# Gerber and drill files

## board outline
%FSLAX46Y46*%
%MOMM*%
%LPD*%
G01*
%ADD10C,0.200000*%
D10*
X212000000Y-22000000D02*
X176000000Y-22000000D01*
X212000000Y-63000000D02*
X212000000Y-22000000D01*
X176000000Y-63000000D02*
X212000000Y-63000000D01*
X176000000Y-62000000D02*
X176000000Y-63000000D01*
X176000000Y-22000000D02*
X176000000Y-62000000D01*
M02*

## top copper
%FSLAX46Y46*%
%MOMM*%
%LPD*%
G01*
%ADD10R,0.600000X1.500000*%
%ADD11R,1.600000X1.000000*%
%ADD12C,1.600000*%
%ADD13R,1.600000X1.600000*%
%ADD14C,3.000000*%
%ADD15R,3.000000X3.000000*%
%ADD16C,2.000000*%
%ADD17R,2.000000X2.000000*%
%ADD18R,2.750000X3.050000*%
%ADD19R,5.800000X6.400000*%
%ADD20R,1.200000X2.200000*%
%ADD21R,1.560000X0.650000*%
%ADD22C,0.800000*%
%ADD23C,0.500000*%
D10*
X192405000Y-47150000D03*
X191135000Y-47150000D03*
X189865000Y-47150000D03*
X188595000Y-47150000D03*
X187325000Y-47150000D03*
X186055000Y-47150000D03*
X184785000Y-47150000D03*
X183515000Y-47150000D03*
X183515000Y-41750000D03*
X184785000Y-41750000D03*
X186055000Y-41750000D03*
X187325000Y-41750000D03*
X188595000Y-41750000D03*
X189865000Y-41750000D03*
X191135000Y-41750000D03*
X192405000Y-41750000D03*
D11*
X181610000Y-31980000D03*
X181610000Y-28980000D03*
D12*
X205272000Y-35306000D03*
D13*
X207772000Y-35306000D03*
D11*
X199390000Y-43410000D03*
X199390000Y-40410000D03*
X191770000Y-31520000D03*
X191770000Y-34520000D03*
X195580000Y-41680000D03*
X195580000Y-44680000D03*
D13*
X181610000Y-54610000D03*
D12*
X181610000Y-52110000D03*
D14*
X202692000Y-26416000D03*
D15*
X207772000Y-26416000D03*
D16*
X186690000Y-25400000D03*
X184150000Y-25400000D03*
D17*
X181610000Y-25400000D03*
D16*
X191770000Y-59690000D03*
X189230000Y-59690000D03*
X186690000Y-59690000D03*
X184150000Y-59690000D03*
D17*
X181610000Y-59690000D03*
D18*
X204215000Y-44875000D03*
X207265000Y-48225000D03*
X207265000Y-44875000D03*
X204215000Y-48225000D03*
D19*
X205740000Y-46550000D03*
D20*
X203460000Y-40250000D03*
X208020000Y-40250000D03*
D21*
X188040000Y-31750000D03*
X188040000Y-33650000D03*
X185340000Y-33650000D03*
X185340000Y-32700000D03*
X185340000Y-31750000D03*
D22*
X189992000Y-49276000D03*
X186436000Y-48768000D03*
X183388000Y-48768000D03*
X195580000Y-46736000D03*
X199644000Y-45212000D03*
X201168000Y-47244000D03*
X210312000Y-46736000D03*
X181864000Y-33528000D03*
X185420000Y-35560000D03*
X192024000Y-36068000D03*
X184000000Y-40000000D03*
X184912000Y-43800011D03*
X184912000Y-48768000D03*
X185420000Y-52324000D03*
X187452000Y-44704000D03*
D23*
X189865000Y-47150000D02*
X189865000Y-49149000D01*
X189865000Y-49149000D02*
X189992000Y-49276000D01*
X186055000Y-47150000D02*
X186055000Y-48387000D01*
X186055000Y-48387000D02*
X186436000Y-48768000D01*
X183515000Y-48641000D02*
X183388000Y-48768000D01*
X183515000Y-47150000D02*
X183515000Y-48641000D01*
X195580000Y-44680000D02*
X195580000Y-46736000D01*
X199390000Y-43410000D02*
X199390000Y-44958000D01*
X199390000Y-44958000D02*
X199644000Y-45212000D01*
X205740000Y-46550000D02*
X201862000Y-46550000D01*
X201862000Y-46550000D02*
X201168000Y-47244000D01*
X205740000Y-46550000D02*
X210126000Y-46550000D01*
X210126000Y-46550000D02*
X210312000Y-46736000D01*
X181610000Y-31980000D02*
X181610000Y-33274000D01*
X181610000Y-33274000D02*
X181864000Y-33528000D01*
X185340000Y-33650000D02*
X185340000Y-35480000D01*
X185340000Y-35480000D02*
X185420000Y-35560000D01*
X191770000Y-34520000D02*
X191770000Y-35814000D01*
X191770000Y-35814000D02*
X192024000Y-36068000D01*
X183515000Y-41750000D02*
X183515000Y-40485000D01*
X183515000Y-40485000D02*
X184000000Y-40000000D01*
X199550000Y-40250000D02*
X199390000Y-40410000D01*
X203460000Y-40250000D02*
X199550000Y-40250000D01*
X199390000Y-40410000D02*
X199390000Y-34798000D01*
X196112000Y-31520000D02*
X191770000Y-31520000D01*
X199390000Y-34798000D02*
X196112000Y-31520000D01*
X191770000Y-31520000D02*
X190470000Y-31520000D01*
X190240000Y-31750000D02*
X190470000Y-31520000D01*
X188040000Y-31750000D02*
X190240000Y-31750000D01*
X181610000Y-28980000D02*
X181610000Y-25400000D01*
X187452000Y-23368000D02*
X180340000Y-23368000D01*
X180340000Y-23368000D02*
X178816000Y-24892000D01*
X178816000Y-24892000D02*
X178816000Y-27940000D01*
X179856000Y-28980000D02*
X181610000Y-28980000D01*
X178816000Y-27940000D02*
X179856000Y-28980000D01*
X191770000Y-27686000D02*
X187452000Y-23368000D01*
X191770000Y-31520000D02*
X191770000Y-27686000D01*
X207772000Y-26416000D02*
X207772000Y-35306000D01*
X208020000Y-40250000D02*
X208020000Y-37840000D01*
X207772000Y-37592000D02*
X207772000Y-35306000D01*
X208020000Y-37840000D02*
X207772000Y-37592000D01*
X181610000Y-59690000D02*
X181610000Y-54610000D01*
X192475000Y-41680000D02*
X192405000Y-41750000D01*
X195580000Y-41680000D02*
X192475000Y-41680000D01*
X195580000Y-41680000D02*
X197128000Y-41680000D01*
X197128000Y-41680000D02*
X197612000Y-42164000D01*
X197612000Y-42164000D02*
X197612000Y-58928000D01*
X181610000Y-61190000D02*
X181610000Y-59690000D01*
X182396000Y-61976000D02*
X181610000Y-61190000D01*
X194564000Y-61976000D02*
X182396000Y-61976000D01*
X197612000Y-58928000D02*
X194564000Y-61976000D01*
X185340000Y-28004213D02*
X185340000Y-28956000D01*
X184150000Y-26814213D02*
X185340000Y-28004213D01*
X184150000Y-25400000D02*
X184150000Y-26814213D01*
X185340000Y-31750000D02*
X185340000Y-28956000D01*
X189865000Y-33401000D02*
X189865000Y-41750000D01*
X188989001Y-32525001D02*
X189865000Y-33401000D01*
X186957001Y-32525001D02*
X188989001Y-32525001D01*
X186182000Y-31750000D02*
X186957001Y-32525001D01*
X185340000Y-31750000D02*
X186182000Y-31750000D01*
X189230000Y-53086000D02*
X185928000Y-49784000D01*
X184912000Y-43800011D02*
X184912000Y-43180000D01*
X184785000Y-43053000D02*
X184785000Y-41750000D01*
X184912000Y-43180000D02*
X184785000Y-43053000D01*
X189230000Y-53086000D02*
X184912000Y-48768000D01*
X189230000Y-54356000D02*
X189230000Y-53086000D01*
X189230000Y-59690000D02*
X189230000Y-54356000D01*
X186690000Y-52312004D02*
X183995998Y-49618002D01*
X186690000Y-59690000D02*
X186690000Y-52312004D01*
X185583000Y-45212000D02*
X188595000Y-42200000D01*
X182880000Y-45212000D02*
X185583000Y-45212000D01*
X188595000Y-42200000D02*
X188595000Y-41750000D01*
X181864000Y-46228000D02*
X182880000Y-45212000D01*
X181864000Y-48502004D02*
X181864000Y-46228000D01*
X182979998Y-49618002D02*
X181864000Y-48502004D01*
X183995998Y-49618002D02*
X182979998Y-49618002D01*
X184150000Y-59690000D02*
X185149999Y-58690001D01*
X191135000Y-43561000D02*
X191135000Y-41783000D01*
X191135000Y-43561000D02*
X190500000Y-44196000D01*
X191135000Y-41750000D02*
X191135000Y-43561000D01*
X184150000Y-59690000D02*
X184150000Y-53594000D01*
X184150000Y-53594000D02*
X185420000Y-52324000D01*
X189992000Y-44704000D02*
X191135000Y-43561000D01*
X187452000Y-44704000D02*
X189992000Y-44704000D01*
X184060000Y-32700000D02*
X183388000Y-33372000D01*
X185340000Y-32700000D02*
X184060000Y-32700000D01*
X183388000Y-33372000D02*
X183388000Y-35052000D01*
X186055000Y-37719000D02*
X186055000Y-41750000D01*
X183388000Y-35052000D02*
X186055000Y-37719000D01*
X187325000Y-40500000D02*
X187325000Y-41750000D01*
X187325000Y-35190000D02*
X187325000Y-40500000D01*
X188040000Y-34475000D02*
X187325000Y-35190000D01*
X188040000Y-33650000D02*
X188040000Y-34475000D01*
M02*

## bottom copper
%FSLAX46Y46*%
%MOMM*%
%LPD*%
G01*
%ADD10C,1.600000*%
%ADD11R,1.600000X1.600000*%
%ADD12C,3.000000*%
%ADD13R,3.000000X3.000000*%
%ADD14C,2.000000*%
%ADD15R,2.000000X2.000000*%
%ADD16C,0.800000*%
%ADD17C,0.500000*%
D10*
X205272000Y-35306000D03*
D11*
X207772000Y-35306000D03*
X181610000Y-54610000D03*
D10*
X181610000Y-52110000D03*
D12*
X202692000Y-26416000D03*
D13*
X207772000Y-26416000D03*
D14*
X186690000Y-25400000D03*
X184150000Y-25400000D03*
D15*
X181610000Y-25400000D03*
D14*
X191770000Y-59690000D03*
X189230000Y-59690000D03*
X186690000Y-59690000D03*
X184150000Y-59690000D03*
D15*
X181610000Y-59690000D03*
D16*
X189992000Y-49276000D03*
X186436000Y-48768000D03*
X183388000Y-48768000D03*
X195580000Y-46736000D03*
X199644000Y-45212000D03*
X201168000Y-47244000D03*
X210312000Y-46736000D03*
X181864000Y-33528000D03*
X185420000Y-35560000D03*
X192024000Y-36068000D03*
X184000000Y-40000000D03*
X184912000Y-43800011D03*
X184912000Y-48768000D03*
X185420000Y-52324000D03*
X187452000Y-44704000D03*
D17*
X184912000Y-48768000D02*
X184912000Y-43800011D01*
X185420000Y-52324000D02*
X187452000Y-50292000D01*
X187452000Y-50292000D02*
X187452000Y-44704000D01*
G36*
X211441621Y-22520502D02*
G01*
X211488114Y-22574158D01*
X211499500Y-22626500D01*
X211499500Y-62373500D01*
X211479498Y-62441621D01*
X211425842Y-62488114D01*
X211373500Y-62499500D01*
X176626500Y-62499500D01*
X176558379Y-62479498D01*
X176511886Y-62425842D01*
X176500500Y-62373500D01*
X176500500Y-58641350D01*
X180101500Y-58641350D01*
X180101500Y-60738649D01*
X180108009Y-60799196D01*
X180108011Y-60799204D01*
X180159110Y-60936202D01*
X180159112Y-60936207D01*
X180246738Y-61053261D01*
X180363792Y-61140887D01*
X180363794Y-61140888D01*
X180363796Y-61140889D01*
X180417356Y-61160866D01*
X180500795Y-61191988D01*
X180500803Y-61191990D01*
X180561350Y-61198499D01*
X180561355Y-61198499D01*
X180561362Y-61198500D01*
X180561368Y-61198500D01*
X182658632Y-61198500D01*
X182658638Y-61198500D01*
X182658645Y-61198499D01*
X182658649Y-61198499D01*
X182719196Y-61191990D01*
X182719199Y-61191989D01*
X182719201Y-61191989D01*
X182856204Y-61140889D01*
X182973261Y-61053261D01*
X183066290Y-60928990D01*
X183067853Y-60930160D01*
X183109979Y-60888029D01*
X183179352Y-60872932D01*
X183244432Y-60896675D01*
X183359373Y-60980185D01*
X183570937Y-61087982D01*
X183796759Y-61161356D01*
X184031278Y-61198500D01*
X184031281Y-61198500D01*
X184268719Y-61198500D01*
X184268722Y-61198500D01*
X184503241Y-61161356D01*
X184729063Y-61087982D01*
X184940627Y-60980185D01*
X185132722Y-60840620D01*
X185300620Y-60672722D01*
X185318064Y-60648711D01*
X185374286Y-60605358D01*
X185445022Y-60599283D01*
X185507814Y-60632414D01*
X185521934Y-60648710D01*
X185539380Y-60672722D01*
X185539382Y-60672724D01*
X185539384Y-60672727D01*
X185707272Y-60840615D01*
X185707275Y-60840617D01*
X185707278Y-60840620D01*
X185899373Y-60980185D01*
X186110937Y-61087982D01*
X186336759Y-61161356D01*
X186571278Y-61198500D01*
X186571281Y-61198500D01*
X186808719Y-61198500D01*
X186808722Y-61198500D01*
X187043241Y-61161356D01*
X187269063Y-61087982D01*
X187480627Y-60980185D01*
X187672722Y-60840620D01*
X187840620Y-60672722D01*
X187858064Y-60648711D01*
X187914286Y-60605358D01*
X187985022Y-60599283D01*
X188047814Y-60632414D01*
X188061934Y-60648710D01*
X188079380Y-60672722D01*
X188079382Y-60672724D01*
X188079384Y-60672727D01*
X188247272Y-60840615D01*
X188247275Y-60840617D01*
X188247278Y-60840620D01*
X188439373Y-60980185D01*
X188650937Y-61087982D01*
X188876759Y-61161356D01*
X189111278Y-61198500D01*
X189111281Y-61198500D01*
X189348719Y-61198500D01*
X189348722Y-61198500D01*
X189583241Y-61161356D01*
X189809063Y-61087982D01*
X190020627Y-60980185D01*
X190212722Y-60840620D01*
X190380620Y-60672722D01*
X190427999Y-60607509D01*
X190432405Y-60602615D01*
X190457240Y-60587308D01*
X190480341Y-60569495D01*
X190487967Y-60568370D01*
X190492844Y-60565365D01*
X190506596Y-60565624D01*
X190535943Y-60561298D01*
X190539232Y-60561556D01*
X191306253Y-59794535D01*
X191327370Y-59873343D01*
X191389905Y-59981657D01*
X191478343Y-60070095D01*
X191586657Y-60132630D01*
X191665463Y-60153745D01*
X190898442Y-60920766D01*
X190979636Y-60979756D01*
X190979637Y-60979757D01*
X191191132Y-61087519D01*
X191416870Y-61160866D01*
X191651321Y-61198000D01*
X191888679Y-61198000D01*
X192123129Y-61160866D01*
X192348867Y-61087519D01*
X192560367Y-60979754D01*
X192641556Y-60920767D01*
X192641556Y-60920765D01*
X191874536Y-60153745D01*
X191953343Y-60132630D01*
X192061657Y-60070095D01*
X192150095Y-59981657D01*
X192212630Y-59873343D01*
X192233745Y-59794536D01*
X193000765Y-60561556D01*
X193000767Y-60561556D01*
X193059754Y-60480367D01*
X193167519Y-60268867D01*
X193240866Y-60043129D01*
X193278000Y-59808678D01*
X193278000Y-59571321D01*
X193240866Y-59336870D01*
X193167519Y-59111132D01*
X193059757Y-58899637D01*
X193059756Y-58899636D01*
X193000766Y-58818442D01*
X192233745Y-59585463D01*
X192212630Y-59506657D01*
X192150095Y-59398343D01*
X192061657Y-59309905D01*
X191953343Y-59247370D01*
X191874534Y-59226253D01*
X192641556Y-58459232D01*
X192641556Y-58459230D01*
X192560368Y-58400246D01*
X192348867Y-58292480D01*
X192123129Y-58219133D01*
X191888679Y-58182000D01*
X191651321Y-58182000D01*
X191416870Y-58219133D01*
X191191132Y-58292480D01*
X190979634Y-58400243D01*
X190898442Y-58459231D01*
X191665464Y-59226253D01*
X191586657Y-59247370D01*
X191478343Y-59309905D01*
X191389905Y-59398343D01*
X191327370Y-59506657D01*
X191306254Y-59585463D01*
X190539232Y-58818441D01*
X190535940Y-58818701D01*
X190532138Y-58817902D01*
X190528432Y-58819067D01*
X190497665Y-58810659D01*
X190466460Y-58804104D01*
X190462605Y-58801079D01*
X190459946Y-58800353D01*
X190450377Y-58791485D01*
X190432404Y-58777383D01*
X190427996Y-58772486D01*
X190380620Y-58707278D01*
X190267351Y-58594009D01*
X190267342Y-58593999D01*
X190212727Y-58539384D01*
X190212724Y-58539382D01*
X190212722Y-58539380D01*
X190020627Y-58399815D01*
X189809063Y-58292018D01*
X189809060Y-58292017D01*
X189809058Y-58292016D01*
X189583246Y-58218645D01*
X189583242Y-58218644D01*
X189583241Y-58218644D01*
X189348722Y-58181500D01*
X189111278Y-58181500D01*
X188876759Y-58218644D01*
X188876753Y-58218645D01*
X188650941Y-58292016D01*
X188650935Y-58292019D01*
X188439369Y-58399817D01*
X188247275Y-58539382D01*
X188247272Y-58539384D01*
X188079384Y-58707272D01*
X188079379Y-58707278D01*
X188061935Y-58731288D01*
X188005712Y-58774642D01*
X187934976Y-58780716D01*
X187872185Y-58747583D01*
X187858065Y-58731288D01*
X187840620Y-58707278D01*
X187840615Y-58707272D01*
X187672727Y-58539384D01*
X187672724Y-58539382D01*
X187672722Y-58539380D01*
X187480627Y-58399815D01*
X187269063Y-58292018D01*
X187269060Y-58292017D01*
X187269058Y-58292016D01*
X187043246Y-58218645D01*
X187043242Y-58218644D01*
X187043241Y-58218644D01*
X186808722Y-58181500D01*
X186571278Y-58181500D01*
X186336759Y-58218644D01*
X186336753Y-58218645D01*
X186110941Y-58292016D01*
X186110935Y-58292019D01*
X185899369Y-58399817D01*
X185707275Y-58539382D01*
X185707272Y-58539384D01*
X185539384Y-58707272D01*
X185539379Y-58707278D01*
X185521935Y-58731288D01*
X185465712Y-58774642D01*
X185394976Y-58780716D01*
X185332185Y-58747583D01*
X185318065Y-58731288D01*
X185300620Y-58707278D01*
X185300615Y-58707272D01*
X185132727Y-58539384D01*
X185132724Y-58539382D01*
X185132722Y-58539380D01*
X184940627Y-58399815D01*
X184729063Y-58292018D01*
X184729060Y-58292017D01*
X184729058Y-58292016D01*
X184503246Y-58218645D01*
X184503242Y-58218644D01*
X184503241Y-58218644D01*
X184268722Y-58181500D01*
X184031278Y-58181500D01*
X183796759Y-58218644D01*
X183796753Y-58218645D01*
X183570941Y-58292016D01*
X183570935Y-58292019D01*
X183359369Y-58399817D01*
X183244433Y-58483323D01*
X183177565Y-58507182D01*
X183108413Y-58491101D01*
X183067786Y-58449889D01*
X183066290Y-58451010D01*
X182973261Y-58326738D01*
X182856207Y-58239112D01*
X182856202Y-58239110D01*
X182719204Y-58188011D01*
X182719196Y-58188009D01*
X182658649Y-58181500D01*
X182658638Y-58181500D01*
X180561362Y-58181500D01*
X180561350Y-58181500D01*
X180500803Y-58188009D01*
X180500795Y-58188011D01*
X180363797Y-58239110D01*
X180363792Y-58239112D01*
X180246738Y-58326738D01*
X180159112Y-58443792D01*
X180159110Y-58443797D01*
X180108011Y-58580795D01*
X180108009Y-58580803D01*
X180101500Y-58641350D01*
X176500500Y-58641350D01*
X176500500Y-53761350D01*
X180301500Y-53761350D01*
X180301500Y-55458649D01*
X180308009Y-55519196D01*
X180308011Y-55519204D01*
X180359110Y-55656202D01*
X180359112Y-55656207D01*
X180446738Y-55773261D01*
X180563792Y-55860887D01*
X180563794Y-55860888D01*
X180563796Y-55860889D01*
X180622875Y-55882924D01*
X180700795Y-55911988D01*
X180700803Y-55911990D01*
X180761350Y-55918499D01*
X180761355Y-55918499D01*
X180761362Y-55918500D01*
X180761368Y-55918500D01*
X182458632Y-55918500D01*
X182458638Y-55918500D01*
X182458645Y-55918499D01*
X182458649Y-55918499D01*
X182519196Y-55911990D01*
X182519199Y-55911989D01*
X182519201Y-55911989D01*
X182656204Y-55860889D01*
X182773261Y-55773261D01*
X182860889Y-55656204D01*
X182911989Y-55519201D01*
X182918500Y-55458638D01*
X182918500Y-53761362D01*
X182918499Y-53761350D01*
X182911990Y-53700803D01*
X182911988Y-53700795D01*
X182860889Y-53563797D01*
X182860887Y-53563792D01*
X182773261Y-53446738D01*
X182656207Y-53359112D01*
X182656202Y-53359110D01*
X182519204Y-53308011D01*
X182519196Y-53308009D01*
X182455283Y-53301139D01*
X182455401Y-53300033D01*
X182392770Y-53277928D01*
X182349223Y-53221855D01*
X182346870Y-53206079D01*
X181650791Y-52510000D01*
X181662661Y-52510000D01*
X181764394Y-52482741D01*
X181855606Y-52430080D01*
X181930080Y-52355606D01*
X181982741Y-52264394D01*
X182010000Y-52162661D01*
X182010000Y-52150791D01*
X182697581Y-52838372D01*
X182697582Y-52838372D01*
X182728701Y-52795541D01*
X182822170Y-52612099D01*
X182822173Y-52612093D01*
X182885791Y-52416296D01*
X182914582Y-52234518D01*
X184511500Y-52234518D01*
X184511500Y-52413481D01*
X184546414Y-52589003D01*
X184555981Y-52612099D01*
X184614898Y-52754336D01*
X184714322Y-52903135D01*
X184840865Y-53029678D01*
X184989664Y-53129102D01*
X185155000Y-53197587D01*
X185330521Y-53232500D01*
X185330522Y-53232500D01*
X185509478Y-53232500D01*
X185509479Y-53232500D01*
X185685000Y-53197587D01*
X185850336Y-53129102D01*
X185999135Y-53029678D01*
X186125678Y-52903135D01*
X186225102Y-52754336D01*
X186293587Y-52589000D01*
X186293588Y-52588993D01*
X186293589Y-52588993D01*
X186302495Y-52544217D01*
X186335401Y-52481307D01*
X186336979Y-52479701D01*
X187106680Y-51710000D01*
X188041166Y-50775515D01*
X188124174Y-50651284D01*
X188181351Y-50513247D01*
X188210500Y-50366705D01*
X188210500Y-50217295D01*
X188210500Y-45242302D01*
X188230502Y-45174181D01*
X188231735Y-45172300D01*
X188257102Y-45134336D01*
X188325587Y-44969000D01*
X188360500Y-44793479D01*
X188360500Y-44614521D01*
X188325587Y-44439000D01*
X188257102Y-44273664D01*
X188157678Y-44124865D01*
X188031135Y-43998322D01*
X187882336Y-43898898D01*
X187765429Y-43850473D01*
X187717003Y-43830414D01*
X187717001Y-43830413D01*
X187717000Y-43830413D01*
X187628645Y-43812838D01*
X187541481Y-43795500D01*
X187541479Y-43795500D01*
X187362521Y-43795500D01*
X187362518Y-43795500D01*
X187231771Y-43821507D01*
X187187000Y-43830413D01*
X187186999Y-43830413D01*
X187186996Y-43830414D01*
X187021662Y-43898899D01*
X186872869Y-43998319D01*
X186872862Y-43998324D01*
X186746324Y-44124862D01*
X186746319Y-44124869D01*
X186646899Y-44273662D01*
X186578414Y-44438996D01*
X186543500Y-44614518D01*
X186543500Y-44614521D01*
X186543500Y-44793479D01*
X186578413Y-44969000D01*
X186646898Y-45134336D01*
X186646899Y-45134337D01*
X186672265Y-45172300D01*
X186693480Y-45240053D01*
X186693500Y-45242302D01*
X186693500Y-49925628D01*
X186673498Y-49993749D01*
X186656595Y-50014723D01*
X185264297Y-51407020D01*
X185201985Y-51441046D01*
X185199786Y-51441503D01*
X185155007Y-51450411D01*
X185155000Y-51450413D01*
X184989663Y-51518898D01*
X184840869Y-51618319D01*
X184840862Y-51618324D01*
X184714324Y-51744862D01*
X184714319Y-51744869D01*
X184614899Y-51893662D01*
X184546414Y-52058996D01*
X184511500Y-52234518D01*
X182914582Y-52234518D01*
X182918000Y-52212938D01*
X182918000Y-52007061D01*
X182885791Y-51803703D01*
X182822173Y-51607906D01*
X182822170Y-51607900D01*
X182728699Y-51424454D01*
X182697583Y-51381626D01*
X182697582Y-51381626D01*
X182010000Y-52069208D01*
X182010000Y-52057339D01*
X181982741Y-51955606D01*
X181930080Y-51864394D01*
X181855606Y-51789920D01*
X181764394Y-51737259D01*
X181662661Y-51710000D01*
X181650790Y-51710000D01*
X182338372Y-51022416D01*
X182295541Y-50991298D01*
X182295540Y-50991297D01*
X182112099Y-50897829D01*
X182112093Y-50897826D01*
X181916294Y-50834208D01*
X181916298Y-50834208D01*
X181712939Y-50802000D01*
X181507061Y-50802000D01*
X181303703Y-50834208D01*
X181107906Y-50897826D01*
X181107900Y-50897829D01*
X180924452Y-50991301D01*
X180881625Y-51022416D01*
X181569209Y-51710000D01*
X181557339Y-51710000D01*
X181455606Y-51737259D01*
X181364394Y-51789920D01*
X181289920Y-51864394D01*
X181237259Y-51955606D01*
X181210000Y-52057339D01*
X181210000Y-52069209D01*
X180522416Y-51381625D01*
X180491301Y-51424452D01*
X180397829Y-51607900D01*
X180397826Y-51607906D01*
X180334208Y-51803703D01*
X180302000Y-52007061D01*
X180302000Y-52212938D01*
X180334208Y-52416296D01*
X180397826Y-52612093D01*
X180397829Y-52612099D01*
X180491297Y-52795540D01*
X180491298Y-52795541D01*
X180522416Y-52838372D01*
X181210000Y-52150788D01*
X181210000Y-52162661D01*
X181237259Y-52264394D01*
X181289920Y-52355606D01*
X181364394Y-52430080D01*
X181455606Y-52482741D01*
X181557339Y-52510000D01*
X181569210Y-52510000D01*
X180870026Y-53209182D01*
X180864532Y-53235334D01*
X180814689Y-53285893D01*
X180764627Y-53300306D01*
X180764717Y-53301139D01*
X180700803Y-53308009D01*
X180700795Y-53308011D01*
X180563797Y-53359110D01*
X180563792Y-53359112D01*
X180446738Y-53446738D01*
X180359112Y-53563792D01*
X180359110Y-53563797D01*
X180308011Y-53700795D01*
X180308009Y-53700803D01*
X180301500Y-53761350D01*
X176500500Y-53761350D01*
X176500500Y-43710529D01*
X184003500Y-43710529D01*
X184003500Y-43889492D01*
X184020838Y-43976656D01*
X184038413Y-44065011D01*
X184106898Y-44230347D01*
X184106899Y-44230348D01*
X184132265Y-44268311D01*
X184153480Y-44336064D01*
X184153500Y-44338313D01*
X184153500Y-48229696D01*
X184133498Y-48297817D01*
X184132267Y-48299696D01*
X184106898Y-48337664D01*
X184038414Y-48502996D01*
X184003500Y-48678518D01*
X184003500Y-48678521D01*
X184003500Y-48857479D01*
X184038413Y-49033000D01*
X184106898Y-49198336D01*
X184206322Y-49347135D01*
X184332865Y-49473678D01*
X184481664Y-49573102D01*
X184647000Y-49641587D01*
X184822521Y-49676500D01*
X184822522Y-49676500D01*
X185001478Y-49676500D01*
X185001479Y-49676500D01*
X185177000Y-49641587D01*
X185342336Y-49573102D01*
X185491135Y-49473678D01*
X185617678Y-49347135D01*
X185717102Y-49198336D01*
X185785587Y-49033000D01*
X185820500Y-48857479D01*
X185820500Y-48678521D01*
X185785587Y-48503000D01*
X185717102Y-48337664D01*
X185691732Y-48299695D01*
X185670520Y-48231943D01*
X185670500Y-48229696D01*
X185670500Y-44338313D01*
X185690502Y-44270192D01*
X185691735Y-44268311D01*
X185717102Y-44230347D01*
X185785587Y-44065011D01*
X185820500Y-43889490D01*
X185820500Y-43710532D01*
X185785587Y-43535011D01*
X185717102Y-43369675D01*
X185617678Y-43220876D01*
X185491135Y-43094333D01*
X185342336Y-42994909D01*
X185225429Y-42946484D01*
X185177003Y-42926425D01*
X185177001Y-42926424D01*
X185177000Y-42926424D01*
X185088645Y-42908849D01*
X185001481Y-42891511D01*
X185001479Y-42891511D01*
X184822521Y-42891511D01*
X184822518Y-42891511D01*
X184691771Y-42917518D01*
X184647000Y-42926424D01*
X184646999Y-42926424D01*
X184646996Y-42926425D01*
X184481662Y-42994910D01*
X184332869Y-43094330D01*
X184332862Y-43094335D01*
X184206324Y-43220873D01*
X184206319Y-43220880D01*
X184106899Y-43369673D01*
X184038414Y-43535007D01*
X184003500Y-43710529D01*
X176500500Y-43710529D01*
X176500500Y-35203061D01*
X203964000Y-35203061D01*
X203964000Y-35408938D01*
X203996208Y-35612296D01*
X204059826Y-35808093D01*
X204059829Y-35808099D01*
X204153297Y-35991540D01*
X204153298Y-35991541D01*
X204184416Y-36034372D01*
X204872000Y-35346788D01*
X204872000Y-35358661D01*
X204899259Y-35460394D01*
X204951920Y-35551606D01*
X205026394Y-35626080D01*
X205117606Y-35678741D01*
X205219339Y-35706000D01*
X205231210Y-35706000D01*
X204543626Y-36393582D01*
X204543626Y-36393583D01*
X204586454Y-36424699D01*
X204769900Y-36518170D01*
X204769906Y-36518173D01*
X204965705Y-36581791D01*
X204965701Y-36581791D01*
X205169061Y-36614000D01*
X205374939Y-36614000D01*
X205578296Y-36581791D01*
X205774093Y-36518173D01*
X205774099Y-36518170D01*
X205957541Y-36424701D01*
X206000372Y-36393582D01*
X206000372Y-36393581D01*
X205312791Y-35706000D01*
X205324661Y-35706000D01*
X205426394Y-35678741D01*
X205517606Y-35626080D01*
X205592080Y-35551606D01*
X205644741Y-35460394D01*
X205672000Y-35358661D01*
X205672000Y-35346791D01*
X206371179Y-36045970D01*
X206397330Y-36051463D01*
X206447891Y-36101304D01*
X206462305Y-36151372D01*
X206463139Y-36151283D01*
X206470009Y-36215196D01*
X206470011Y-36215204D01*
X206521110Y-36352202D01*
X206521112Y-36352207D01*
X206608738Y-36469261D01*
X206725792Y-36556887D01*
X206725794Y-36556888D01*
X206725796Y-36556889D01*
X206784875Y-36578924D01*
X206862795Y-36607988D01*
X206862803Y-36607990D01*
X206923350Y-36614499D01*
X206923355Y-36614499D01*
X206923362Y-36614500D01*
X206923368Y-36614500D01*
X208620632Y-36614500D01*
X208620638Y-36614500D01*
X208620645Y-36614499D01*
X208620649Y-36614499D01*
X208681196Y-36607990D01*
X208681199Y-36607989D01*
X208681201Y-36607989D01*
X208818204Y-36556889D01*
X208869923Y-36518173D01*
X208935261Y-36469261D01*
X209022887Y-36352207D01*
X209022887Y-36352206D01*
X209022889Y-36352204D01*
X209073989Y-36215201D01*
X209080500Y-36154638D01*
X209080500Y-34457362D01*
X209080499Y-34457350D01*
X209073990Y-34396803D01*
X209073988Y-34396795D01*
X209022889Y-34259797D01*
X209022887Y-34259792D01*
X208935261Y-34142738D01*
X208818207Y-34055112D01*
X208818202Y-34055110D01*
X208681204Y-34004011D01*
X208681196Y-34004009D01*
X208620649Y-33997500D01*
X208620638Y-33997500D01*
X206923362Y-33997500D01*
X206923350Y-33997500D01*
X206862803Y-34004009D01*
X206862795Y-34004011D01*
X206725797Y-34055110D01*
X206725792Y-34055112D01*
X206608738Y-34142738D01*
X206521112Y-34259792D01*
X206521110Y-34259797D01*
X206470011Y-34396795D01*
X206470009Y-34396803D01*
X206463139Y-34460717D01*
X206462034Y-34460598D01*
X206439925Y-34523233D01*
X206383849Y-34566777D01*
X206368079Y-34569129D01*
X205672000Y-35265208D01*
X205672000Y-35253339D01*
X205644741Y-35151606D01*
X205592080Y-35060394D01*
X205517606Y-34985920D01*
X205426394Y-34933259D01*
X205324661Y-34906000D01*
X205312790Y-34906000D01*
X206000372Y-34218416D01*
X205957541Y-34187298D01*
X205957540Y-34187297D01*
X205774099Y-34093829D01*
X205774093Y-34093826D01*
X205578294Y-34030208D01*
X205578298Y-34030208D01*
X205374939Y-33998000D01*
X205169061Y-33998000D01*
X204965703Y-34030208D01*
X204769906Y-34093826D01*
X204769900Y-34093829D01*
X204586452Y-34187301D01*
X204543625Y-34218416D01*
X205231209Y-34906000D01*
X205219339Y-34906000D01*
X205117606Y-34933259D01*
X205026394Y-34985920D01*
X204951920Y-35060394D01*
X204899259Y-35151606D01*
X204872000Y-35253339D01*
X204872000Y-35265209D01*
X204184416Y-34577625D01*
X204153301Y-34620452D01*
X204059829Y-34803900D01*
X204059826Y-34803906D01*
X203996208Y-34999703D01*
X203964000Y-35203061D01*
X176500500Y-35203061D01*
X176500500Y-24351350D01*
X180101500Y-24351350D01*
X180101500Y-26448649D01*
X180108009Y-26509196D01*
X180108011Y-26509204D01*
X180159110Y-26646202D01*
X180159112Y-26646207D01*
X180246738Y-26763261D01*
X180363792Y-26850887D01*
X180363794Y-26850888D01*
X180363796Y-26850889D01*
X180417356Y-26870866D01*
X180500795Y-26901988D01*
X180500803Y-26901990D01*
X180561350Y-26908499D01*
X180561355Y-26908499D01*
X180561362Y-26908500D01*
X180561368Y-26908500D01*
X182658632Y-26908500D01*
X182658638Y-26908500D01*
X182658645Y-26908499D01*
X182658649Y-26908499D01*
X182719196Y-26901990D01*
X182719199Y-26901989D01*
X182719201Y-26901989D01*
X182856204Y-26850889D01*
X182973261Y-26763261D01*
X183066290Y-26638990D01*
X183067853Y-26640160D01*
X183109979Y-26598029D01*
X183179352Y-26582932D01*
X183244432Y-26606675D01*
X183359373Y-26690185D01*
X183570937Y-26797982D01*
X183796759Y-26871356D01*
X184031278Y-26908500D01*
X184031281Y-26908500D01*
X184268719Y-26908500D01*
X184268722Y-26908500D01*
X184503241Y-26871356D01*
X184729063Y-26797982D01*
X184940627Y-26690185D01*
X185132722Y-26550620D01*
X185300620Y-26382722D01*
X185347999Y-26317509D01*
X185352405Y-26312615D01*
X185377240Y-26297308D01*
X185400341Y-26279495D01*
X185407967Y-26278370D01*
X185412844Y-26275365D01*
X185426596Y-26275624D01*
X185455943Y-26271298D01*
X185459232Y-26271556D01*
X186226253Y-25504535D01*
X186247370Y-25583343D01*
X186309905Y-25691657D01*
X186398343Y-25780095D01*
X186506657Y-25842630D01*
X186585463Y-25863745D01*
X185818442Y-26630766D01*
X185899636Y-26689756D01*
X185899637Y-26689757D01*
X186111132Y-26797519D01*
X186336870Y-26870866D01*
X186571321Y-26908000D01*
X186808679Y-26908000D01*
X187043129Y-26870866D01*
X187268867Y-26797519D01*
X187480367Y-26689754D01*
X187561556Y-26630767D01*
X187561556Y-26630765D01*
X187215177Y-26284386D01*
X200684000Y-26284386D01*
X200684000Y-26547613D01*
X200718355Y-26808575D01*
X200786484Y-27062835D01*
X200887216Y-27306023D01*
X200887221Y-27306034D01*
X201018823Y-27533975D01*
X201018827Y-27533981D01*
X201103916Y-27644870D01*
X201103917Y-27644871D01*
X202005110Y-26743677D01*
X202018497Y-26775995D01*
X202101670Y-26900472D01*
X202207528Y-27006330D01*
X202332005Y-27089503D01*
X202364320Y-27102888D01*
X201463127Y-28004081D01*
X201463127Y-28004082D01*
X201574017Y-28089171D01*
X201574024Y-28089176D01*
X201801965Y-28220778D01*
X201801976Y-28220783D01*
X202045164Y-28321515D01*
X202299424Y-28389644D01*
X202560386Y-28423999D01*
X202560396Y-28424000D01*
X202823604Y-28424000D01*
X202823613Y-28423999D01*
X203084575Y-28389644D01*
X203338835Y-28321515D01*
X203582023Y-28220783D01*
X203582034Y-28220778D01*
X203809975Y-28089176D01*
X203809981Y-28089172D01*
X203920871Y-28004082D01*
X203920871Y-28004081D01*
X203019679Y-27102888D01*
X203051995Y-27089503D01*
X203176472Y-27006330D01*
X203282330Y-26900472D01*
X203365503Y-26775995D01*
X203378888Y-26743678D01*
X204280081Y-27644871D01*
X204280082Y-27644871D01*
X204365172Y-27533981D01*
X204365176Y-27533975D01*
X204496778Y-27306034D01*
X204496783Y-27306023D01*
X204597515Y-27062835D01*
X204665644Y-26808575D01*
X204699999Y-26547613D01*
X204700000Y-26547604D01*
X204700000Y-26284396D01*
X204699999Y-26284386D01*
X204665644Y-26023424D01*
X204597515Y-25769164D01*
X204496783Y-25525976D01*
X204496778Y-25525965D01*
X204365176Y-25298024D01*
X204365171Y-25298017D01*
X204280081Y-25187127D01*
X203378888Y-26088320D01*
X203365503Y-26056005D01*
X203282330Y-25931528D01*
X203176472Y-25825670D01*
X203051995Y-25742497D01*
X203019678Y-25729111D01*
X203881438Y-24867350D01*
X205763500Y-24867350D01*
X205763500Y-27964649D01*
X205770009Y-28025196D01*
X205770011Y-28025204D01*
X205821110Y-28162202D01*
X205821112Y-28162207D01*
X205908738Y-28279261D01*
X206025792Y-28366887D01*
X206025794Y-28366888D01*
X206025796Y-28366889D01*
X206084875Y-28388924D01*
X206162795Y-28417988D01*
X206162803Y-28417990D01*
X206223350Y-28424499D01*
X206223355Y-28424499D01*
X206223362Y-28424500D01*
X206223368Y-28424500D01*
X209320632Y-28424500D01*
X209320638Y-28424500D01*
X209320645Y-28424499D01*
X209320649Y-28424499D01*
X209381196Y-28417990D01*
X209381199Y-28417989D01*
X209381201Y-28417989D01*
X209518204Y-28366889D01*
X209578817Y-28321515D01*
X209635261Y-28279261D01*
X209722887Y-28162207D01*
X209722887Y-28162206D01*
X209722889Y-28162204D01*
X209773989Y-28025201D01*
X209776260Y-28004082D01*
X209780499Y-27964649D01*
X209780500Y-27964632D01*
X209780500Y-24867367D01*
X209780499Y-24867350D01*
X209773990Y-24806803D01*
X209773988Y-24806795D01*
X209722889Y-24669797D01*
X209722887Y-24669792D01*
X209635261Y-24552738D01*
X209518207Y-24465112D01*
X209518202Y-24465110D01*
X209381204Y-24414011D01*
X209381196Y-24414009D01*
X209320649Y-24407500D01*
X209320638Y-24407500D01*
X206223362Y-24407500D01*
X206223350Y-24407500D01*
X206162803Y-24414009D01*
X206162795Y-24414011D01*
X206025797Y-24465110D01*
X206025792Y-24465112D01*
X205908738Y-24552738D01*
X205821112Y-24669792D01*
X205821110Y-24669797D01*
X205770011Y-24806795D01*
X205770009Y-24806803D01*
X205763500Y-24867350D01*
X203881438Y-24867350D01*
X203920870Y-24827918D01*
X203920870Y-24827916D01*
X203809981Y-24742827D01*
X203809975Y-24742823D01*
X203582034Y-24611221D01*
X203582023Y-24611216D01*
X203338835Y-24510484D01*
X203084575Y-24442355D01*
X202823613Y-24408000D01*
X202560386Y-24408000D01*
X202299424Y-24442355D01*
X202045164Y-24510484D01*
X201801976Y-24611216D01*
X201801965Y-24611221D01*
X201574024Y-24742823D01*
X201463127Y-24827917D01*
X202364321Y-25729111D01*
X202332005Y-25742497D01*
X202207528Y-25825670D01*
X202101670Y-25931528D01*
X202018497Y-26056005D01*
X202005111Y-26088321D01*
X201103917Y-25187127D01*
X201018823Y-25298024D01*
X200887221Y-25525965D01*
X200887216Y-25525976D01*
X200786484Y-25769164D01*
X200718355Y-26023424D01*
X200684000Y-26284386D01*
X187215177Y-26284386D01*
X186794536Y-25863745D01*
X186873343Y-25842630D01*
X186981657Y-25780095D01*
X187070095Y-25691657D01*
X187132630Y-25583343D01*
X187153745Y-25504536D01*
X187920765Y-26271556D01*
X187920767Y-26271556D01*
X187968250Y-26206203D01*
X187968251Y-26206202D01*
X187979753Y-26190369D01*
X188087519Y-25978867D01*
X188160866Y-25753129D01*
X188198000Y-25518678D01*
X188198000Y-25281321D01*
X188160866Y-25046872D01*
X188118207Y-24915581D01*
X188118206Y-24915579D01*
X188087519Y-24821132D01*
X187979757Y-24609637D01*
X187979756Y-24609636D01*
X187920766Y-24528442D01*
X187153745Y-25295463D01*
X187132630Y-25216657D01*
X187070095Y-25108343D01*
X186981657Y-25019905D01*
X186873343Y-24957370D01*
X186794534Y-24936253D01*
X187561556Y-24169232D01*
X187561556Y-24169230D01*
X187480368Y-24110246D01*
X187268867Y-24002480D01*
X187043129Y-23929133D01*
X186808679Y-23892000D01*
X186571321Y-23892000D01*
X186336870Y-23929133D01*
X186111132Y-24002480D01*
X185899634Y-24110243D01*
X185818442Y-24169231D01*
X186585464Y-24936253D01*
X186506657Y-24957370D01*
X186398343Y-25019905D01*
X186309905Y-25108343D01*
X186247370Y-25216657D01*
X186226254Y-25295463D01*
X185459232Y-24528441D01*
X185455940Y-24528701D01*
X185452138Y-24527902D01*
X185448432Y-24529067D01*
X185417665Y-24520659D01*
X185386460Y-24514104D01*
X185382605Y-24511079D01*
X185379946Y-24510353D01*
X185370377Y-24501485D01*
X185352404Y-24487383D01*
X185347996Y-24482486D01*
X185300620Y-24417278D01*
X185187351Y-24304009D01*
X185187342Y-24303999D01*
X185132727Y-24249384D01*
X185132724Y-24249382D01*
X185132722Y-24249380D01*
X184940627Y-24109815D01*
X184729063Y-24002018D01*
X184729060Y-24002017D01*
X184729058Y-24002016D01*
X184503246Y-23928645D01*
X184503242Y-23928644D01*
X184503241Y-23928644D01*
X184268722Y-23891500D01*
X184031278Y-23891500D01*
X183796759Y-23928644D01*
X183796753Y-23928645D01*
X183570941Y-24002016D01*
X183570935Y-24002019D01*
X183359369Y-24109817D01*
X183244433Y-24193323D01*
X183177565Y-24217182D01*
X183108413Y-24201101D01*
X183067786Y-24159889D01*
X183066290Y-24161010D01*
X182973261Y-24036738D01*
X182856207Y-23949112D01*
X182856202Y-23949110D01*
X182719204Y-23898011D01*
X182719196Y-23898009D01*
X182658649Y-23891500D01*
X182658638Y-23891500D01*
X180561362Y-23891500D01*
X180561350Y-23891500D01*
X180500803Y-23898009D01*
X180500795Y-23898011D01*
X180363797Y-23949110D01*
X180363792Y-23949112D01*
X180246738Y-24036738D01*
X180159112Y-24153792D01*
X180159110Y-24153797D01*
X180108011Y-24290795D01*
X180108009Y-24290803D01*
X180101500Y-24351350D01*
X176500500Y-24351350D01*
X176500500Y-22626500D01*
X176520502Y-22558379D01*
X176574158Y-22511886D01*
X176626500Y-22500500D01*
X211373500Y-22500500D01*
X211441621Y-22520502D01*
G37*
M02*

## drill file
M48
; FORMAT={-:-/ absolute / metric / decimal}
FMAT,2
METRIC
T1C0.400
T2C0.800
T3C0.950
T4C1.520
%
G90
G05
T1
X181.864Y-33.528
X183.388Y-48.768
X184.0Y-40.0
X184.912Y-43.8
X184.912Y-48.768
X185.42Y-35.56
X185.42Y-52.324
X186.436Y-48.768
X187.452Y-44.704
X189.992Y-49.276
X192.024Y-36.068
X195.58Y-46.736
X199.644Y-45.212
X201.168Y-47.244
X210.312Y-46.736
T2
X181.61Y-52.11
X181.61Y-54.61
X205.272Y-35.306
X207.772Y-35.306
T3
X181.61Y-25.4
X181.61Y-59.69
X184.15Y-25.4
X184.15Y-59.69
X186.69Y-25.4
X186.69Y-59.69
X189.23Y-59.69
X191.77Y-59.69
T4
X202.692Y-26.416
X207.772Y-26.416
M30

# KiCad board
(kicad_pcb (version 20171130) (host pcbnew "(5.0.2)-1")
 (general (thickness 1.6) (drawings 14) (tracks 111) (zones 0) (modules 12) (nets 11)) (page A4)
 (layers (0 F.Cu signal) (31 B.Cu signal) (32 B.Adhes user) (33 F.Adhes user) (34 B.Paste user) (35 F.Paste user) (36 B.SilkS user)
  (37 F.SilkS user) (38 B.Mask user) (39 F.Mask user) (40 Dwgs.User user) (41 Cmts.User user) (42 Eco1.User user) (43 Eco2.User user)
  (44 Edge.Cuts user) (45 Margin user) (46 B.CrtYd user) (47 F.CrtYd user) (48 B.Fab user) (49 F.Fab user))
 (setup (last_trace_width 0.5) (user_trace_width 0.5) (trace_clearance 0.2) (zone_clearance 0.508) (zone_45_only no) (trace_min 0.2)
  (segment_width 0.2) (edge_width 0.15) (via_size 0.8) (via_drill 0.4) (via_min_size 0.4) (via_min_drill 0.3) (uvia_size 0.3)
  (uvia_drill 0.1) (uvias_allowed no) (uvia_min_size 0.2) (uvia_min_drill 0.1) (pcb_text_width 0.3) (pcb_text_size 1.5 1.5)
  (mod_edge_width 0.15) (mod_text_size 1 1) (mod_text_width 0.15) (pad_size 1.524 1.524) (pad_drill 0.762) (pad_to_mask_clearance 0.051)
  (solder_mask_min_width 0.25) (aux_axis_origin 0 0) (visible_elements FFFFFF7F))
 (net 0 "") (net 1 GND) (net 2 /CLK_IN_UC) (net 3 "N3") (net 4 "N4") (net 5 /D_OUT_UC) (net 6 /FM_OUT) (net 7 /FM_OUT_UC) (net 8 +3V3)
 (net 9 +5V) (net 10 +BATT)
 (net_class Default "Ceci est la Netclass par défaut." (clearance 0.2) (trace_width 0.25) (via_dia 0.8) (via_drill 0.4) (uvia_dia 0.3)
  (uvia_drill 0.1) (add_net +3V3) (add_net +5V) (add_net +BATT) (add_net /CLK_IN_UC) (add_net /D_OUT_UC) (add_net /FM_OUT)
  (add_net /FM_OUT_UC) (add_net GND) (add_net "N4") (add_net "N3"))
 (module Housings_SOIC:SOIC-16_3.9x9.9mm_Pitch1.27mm (layer F.Cu) (at 187.96 44.45 270)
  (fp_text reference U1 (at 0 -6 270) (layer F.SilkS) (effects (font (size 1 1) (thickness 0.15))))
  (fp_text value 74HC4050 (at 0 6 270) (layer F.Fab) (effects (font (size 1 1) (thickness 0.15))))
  (pad 16 smd rect (at 2.7 -4.445 270) (size 1.5 0.6) (layers F.Cu F.Paste F.Mask))
  (pad 15 smd rect (at 2.7 -3.175 270) (size 1.5 0.6) (layers F.Cu F.Paste F.Mask))
  (pad 14 smd rect (at 2.7 -1.905 270) (size 1.5 0.6) (layers F.Cu F.Paste F.Mask) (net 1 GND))
  (pad 13 smd rect (at 2.7 -0.635 270) (size 1.5 0.6) (layers F.Cu F.Paste F.Mask))
  (pad 12 smd rect (at 2.7 0.635 270) (size 1.5 0.6) (layers F.Cu F.Paste F.Mask))
  (pad 11 smd rect (at 2.7 1.905 270) (size 1.5 0.6) (layers F.Cu F.Paste F.Mask) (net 1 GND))
  (pad 10 smd rect (at 2.7 3.175 270) (size 1.5 0.6) (layers F.Cu F.Paste F.Mask))
  (pad 9 smd rect (at 2.7 4.445 270) (size 1.5 0.6) (layers F.Cu F.Paste F.Mask) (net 1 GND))
  (pad 8 smd rect (at -2.7 4.445 270) (size 1.5 0.6) (layers F.Cu F.Paste F.Mask) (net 1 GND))
  (pad 7 smd rect (at -2.7 3.175 270) (size 1.5 0.6) (layers F.Cu F.Paste F.Mask) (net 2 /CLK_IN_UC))
  (pad 6 smd rect (at -2.7 1.905 270) (size 1.5 0.6) (layers F.Cu F.Paste F.Mask) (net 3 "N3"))
  (pad 5 smd rect (at -2.7 0.635 270) (size 1.5 0.6) (layers F.Cu F.Paste F.Mask) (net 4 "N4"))
  (pad 4 smd rect (at -2.7 -0.635 270) (size 1.5 0.6) (layers F.Cu F.Paste F.Mask) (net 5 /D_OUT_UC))
  (pad 3 smd rect (at -2.7 -1.905 270) (size 1.5 0.6) (layers F.Cu F.Paste F.Mask) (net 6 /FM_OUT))
  (pad 2 smd rect (at -2.7 -3.175 270) (size 1.5 0.6) (layers F.Cu F.Paste F.Mask) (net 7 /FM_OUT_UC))
  (pad 1 smd rect (at -2.7 -4.445 270) (size 1.5 0.6) (layers F.Cu F.Paste F.Mask) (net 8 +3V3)))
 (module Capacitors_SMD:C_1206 (layer F.Cu) (at 181.61 30.48 270)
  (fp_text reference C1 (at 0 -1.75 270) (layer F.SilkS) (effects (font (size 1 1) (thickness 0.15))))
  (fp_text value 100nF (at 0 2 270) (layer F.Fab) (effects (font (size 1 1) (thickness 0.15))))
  (pad 2 smd rect (at 1.5 0 270) (size 1 1.6) (layers F.Cu F.Paste F.Mask) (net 1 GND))
  (pad 1 smd rect (at -1.5 0 270) (size 1 1.6) (layers F.Cu F.Paste F.Mask) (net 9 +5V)))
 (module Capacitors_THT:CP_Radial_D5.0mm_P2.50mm (layer F.Cu) (at 207.772 35.306 180)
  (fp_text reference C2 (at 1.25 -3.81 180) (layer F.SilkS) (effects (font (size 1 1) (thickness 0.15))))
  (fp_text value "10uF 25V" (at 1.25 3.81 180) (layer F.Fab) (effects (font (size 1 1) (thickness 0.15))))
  (pad 2 thru_hole circle (at 2.5 0 180) (size 1.6 1.6) (drill 0.8) (layers *.Cu *.Mask) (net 1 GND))
  (pad 1 thru_hole rect (at 0 0 180) (size 1.6 1.6) (drill 0.8) (layers *.Cu *.Mask) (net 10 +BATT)))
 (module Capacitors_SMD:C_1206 (layer F.Cu) (at 199.39 41.91 270)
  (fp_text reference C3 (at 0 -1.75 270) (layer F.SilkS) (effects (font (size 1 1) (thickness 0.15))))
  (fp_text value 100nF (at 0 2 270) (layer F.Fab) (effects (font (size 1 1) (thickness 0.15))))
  (pad 2 smd rect (at 1.5 0 270) (size 1 1.6) (layers F.Cu F.Paste F.Mask) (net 1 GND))
  (pad 1 smd rect (at -1.5 0 270) (size 1 1.6) (layers F.Cu F.Paste F.Mask) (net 9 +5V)))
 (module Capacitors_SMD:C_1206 (layer F.Cu) (at 191.77 33.02 270)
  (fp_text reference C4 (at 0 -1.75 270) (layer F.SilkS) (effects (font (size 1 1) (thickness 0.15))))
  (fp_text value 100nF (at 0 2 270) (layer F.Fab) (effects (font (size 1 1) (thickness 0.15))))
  (pad 1 smd rect (at -1.5 0 270) (size 1 1.6) (layers F.Cu F.Paste F.Mask) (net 9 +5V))
  (pad 2 smd rect (at 1.5 0 270) (size 1 1.6) (layers F.Cu F.Paste F.Mask) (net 1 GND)))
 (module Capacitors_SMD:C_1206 (layer F.Cu) (at 195.58 43.18 270)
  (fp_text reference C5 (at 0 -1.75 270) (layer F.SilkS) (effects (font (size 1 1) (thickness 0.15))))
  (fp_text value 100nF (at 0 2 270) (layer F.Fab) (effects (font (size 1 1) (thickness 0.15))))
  (pad 1 smd rect (at -1.5 0 270) (size 1 1.6) (layers F.Cu F.Paste F.Mask) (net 8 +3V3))
  (pad 2 smd rect (at 1.5 0 270) (size 1 1.6) (layers F.Cu F.Paste F.Mask) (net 1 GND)))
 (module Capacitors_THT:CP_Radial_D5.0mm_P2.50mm (layer F.Cu) (at 181.61 54.61 90)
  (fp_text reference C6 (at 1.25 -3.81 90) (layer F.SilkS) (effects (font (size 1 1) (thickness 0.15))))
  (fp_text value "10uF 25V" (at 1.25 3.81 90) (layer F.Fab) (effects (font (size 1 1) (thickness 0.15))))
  (pad 1 thru_hole rect (at 0 0 90) (size 1.6 1.6) (drill 0.8) (layers *.Cu *.Mask) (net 8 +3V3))
  (pad 2 thru_hole circle (at 2.5 0 90) (size 1.6 1.6) (drill 0.8) (layers *.Cu *.Mask) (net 1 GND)))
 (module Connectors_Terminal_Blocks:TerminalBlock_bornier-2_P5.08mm (layer F.Cu) (at 207.772 26.416 180)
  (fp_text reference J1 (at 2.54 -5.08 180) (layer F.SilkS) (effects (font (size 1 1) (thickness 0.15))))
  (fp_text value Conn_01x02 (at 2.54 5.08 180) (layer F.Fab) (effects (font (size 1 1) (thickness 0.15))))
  (pad 2 thru_hole circle (at 5.08 0 180) (size 3 3) (drill 1.52) (layers *.Cu *.Mask) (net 1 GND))
  (pad 1 thru_hole rect (at 0 0 180) (size 3 3) (drill 1.52) (layers *.Cu *.Mask) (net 10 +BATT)))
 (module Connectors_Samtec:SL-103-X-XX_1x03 (layer F.Cu) (at 181.61 25.4 90)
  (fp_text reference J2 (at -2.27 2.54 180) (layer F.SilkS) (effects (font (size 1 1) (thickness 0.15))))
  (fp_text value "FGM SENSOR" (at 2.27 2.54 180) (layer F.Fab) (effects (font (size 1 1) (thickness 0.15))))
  (pad 3 thru_hole circle (at 0 5.08 90) (size 2 2) (drill 0.95) (layers *.Cu *.Mask) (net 1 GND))
  (pad 2 thru_hole circle (at 0 2.54 90) (size 2 2) (drill 0.95) (layers *.Cu *.Mask) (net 6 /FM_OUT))
  (pad 1 thru_hole rect (at 0 0 90) (size 2 2) (drill 0.95) (layers *.Cu *.Mask) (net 9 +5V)))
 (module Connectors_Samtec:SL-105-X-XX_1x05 (layer F.Cu) (at 181.61 59.69 90)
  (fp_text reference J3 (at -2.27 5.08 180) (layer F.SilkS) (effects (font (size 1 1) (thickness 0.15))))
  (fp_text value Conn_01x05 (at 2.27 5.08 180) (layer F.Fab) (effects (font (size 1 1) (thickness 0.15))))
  (pad 5 thru_hole circle (at 0 10.16 90) (size 2 2) (drill 0.95) (layers *.Cu *.Mask) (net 1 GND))
  (pad 4 thru_hole circle (at 0 7.62 90) (size 2 2) (drill 0.95) (layers *.Cu *.Mask) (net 2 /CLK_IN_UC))
  (pad 3 thru_hole circle (at 0 5.08 90) (size 2 2) (drill 0.95) (layers *.Cu *.Mask) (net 5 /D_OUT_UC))
  (pad 2 thru_hole circle (at 0 2.54 90) (size 2 2) (drill 0.95) (layers *.Cu *.Mask) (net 7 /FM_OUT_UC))
  (pad 1 thru_hole rect (at 0 0 90) (size 2 2) (drill 0.95) (layers *.Cu *.Mask) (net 8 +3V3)))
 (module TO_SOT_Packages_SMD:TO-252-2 (layer F.Cu) (at 205.74 44.45 270)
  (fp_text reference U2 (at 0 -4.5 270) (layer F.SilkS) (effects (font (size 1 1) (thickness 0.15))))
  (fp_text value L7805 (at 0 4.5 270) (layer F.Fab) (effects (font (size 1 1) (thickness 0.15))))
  (pad 2 smd rect (at 0.425 1.525 270) (size 3.05 2.75) (layers F.Cu F.Paste) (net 1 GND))
  (pad 2 smd rect (at 3.775 -1.525 270) (size 3.05 2.75) (layers F.Cu F.Paste) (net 1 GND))
  (pad 2 smd rect (at 0.425 -1.525 270) (size 3.05 2.75) (layers F.Cu F.Paste) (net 1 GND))
  (pad 2 smd rect (at 3.775 1.525 270) (size 3.05 2.75) (layers F.Cu F.Paste) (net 1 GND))
  (pad 2 smd rect (at 2.1 0 270) (size 6.4 5.8) (layers F.Cu F.Mask) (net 1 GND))
  (pad 3 smd rect (at -4.2 2.28 270) (size 2.2 1.2) (layers F.Cu F.Paste F.Mask) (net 9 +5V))
  (pad 1 smd rect (at -4.2 -2.28 270) (size 2.2 1.2) (layers F.Cu F.Paste F.Mask) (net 10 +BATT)))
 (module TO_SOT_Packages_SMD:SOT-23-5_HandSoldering (layer F.Cu) (at 186.69 32.7)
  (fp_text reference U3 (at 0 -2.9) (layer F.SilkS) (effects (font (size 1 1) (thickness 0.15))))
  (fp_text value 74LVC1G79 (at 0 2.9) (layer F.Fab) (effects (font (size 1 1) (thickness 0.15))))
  (pad 5 smd rect (at 1.35 -0.95) (size 1.56 0.65) (layers F.Cu F.Paste F.Mask) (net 9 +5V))
  (pad 4 smd rect (at 1.35 0.95) (size 1.56 0.65) (layers F.Cu F.Paste F.Mask) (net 4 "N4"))
  (pad 3 smd rect (at -1.35 0.95) (size 1.56 0.65) (layers F.Cu F.Paste F.Mask) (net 1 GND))
  (pad 2 smd rect (at -1.35 0) (size 1.56 0.65) (layers F.Cu F.Paste F.Mask) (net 3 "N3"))
  (pad 1 smd rect (at -1.35 -0.95) (size 1.56 0.65) (layers F.Cu F.Paste F.Mask) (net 6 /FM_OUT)))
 (gr_line (start 212 22) (end 176 22) (layer Edge.Cuts) (width 0.2))
 (gr_line (start 212 63) (end 212 22) (layer Edge.Cuts) (width 0.2))
 (gr_line (start 176 63) (end 212 63) (layer Edge.Cuts) (width 0.2))
 (gr_line (start 176 62) (end 176 63) (layer Edge.Cuts) (width 0.2))
 (gr_line (start 176 22) (end 176 62) (layer Edge.Cuts) (width 0.2))
 (via (at 189.992 49.276) (size 0.8) (drill 0.4) (layers F.Cu B.Cu) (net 1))
 (segment (start 189.865 47.15) (end 189.865 49.149) (width 0.5) (layer F.Cu) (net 1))
 (segment (start 189.865 49.149) (end 189.992 49.276) (width 0.5) (layer F.Cu) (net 1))
 (via (at 186.436 48.768) (size 0.8) (drill 0.4) (layers F.Cu B.Cu) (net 1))
 (segment (start 186.055 47.15) (end 186.055 48.387) (width 0.5) (layer F.Cu) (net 1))
 (segment (start 186.055 48.387) (end 186.436 48.768) (width 0.5) (layer F.Cu) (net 1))
 (segment (start 183.515 48.641) (end 183.388 48.768) (width 0.5) (layer F.Cu) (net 1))
 (segment (start 183.515 47.15) (end 183.515 48.641) (width 0.5) (layer F.Cu) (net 1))
 (via (at 183.388 48.768) (size 0.8) (drill 0.4) (layers F.Cu B.Cu) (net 1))
 (via (at 195.58 46.736) (size 0.8) (drill 0.4) (layers F.Cu B.Cu) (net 1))
 (segment (start 195.58 44.68) (end 195.58 46.736) (width 0.5) (layer F.Cu) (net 1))
 (via (at 199.644 45.212) (size 0.8) (drill 0.4) (layers F.Cu B.Cu) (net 1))
 (segment (start 199.39 43.41) (end 199.39 44.958) (width 0.5) (layer F.Cu) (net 1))
 (segment (start 199.39 44.958) (end 199.644 45.212) (width 0.5) (layer F.Cu) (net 1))
 (via (at 201.168 47.244) (size 0.8) (drill 0.4) (layers F.Cu B.Cu) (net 1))
 (segment (start 205.74 46.55) (end 201.862 46.55) (width 0.5) (layer F.Cu) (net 1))
 (segment (start 201.862 46.55) (end 201.168 47.244) (width 0.5) (layer F.Cu) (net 1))
 (via (at 210.312 46.736) (size 0.8) (drill 0.4) (layers F.Cu B.Cu) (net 1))
 (segment (start 205.74 46.55) (end 210.126 46.55) (width 0.5) (layer F.Cu) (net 1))
 (segment (start 210.126 46.55) (end 210.312 46.736) (width 0.5) (layer F.Cu) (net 1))
 (via (at 181.864 33.528) (size 0.8) (drill 0.4) (layers F.Cu B.Cu) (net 1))
 (segment (start 181.61 31.98) (end 181.61 33.274) (width 0.5) (layer F.Cu) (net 1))
 (segment (start 181.61 33.274) (end 181.864 33.528) (width 0.5) (layer F.Cu) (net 1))
 (via (at 185.42 35.56) (size 0.8) (drill 0.4) (layers F.Cu B.Cu) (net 1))
 (segment (start 185.34 33.65) (end 185.34 35.48) (width 0.5) (layer F.Cu) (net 1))
 (segment (start 185.34 35.48) (end 185.42 35.56) (width 0.5) (layer F.Cu) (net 1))
 (via (at 192.024 36.068) (size 0.8) (drill 0.4) (layers F.Cu B.Cu) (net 1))
 (segment (start 191.77 34.52) (end 191.77 35.814) (width 0.5) (layer F.Cu) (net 1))
 (segment (start 191.77 35.814) (end 192.024 36.068) (width 0.5) (layer F.Cu) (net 1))
 (via (at 184 40) (size 0.8) (drill 0.4) (layers F.Cu B.Cu) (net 1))
 (segment (start 183.515 41.75) (end 183.515 40.485) (width 0.5) (layer F.Cu) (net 1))
 (segment (start 183.515 40.485) (end 184 40) (width 0.5) (layer F.Cu) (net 1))
 (segment (start 199.55 40.25) (end 199.39 40.41) (width 0.5) (layer F.Cu) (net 9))
 (segment (start 203.46 40.25) (end 199.55 40.25) (width 0.5) (layer F.Cu) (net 9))
 (segment (start 199.39 40.41) (end 199.39 34.798) (width 0.5) (layer F.Cu) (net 9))
 (segment (start 196.112 31.52) (end 191.77 31.52) (width 0.5) (layer F.Cu) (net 9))
 (segment (start 199.39 34.798) (end 196.112 31.52) (width 0.5) (layer F.Cu) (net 9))
 (segment (start 191.77 31.52) (end 190.47 31.52) (width 0.5) (layer F.Cu) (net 9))
 (segment (start 190.24 31.75) (end 190.47 31.52) (width 0.5) (layer F.Cu) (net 9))
 (segment (start 188.04 31.75) (end 190.24 31.75) (width 0.5) (layer F.Cu) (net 9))
 (segment (start 181.61 28.98) (end 181.61 25.4) (width 0.5) (layer F.Cu) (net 9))
 (segment (start 187.452 23.368) (end 180.34 23.368) (width 0.5) (layer F.Cu) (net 9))
 (segment (start 180.34 23.368) (end 178.816 24.892) (width 0.5) (layer F.Cu) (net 9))
 (segment (start 178.816 24.892) (end 178.816 27.94) (width 0.5) (layer F.Cu) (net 9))
 (segment (start 179.856 28.98) (end 181.61 28.98) (width 0.5) (layer F.Cu) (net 9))
 (segment (start 178.816 27.94) (end 179.856 28.98) (width 0.5) (layer F.Cu) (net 9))
 (segment (start 191.77 27.686) (end 187.452 23.368) (width 0.5) (layer F.Cu) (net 9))
 (segment (start 191.77 31.52) (end 191.77 27.686) (width 0.5) (layer F.Cu) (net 9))
 (segment (start 207.772 26.416) (end 207.772 35.306) (width 0.5) (layer F.Cu) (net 10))
 (segment (start 208.02 40.25) (end 208.02 37.84) (width 0.5) (layer F.Cu) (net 10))
 (segment (start 207.772 37.592) (end 207.772 35.306) (width 0.5) (layer F.Cu) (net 10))
 (segment (start 208.02 37.84) (end 207.772 37.592) (width 0.5) (layer F.Cu) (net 10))
 (segment (start 181.61 59.69) (end 181.61 54.61) (width 0.5) (layer F.Cu) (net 8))
 (segment (start 192.475 41.68) (end 192.405 41.75) (width 0.5) (layer F.Cu) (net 8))
 (segment (start 195.58 41.68) (end 192.475 41.68) (width 0.5) (layer F.Cu) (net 8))
 (segment (start 195.58 41.68) (end 197.128 41.68) (width 0.5) (layer F.Cu) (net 8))
 (segment (start 197.128 41.68) (end 197.612 42.164) (width 0.5) (layer F.Cu) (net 8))
 (segment (start 197.612 42.164) (end 197.612 58.928) (width 0.5) (layer F.Cu) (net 8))
 (segment (start 181.61 61.19) (end 181.61 59.69) (width 0.5) (layer F.Cu) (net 8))
 (segment (start 182.396 61.976) (end 181.61 61.19) (width 0.5) (layer F.Cu) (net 8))
 (segment (start 194.564 61.976) (end 182.396 61.976) (width 0.5) (layer F.Cu) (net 8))
 (segment (start 197.612 58.928) (end 194.564 61.976) (width 0.5) (layer F.Cu) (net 8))
 (segment (start 185.34 28.004213) (end 185.34 28.956) (width 0.5) (layer F.Cu) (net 6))
 (segment (start 184.15 26.814213) (end 185.34 28.004213) (width 0.5) (layer F.Cu) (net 6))
 (segment (start 184.15 25.4) (end 184.15 26.814213) (width 0.5) (layer F.Cu) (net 6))
 (segment (start 185.34 31.75) (end 185.34 28.956) (width 0.5) (layer F.Cu) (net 6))
 (segment (start 189.865 33.401) (end 189.865 41.75) (width 0.5) (layer F.Cu) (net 6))
 (segment (start 188.989001 32.525001) (end 189.865 33.401) (width 0.5) (layer F.Cu) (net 6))
 (segment (start 186.957001 32.525001) (end 188.989001 32.525001) (width 0.5) (layer F.Cu) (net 6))
 (segment (start 186.182 31.75) (end 186.957001 32.525001) (width 0.5) (layer F.Cu) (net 6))
 (segment (start 185.34 31.75) (end 186.182 31.75) (width 0.5) (layer F.Cu) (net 6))
 (segment (start 189.23 53.086) (end 185.928 49.784) (width 0.5) (layer F.Cu) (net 2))
 (via (at 184.912 43.800011) (size 0.8) (drill 0.4) (layers F.Cu B.Cu) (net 2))
 (segment (start 184.912 48.768) (end 184.912 43.800011) (width 0.5) (layer B.Cu) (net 2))
 (segment (start 184.912 43.800011) (end 184.912 43.18) (width 0.5) (layer F.Cu) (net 2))
 (segment (start 184.785 43.053) (end 184.785 41.75) (width 0.5) (layer F.Cu) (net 2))
 (segment (start 184.912 43.18) (end 184.785 43.053) (width 0.5) (layer F.Cu) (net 2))
 (via (at 184.912 48.768) (size 0.8) (drill 0.4) (layers F.Cu B.Cu) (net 2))
 (segment (start 189.23 53.086) (end 184.912 48.768) (width 0.5) (layer F.Cu) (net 2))
 (segment (start 189.23 54.356) (end 189.23 53.086) (width 0.5) (layer F.Cu) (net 2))
 (segment (start 189.23 59.69) (end 189.23 54.356) (width 0.5) (layer F.Cu) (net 2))
 (segment (start 186.69 52.312004) (end 183.995998 49.618002) (width 0.5) (layer F.Cu) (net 5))
 (segment (start 186.69 59.69) (end 186.69 52.312004) (width 0.5) (layer F.Cu) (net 5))
 (segment (start 185.583 45.212) (end 188.595 42.2) (width 0.5) (layer F.Cu) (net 5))
 (segment (start 182.88 45.212) (end 185.583 45.212) (width 0.5) (layer F.Cu) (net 5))
 (segment (start 188.595 42.2) (end 188.595 41.75) (width 0.5) (layer F.Cu) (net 5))
 (segment (start 181.864 46.228) (end 182.88 45.212) (width 0.5) (layer F.Cu) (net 5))
 (segment (start 181.864 48.502004) (end 181.864 46.228) (width 0.5) (layer F.Cu) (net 5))
 (segment (start 182.979998 49.618002) (end 181.864 48.502004) (width 0.5) (layer F.Cu) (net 5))
 (segment (start 183.995998 49.618002) (end 182.979998 49.618002) (width 0.5) (layer F.Cu) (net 5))
 (segment (start 184.15 59.69) (end 185.149999 58.690001) (width 0.5) (layer F.Cu) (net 7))
 (segment (start 191.135 43.561) (end 191.135 41.783) (width 0.5) (layer F.Cu) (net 7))
 (segment (start 191.135 43.561) (end 190.5 44.196) (width 0.5) (layer F.Cu) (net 7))
 (segment (start 191.135 41.75) (end 191.135 43.561) (width 0.5) (layer F.Cu) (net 7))
 (via (at 185.42 52.324) (size 0.8) (drill 0.4) (layers F.Cu B.Cu) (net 7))
 (segment (start 184.15 59.69) (end 184.15 53.594) (width 0.5) (layer F.Cu) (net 7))
 (segment (start 184.15 53.594) (end 185.42 52.324) (width 0.5) (layer F.Cu) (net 7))
 (via (at 187.452 44.704) (size 0.8) (drill 0.4) (layers F.Cu B.Cu) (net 7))
 (segment (start 185.42 52.324) (end 187.452 50.292) (width 0.5) (layer B.Cu) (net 7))
 (segment (start 187.452 50.292) (end 187.452 44.704) (width 0.5) (layer B.Cu) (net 7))
 (segment (start 189.992 44.704) (end 191.135 43.561) (width 0.5) (layer F.Cu) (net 7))
 (segment (start 187.452 44.704) (end 189.992 44.704) (width 0.5) (layer F.Cu) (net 7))
 (segment (start 184.06 32.7) (end 183.388 33.372) (width 0.5) (layer F.Cu) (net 3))
 (segment (start 185.34 32.7) (end 184.06 32.7) (width 0.5) (layer F.Cu) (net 3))
 (segment (start 183.388 33.372) (end 183.388 35.052) (width 0.5) (layer F.Cu) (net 3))
 (segment (start 186.055 37.719) (end 186.055 41.75) (width 0.5) (layer F.Cu) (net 3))
 (segment (start 183.388 35.052) (end 186.055 37.719) (width 0.5) (layer F.Cu) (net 3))
 (segment (start 187.325 40.5) (end 187.325 41.75) (width 0.5) (layer F.Cu) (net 4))
 (segment (start 187.325 35.19) (end 187.325 40.5) (width 0.5) (layer F.Cu) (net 4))
 (segment (start 188.04 34.475) (end 187.325 35.19) (width 0.5) (layer F.Cu) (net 4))
 (segment (start 188.04 33.65) (end 188.04 34.475) (width 0.5) (layer F.Cu) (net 4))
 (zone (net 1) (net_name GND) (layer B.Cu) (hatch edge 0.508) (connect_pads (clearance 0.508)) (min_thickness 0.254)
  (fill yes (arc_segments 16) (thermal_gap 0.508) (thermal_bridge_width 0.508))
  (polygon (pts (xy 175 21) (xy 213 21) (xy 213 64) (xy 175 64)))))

